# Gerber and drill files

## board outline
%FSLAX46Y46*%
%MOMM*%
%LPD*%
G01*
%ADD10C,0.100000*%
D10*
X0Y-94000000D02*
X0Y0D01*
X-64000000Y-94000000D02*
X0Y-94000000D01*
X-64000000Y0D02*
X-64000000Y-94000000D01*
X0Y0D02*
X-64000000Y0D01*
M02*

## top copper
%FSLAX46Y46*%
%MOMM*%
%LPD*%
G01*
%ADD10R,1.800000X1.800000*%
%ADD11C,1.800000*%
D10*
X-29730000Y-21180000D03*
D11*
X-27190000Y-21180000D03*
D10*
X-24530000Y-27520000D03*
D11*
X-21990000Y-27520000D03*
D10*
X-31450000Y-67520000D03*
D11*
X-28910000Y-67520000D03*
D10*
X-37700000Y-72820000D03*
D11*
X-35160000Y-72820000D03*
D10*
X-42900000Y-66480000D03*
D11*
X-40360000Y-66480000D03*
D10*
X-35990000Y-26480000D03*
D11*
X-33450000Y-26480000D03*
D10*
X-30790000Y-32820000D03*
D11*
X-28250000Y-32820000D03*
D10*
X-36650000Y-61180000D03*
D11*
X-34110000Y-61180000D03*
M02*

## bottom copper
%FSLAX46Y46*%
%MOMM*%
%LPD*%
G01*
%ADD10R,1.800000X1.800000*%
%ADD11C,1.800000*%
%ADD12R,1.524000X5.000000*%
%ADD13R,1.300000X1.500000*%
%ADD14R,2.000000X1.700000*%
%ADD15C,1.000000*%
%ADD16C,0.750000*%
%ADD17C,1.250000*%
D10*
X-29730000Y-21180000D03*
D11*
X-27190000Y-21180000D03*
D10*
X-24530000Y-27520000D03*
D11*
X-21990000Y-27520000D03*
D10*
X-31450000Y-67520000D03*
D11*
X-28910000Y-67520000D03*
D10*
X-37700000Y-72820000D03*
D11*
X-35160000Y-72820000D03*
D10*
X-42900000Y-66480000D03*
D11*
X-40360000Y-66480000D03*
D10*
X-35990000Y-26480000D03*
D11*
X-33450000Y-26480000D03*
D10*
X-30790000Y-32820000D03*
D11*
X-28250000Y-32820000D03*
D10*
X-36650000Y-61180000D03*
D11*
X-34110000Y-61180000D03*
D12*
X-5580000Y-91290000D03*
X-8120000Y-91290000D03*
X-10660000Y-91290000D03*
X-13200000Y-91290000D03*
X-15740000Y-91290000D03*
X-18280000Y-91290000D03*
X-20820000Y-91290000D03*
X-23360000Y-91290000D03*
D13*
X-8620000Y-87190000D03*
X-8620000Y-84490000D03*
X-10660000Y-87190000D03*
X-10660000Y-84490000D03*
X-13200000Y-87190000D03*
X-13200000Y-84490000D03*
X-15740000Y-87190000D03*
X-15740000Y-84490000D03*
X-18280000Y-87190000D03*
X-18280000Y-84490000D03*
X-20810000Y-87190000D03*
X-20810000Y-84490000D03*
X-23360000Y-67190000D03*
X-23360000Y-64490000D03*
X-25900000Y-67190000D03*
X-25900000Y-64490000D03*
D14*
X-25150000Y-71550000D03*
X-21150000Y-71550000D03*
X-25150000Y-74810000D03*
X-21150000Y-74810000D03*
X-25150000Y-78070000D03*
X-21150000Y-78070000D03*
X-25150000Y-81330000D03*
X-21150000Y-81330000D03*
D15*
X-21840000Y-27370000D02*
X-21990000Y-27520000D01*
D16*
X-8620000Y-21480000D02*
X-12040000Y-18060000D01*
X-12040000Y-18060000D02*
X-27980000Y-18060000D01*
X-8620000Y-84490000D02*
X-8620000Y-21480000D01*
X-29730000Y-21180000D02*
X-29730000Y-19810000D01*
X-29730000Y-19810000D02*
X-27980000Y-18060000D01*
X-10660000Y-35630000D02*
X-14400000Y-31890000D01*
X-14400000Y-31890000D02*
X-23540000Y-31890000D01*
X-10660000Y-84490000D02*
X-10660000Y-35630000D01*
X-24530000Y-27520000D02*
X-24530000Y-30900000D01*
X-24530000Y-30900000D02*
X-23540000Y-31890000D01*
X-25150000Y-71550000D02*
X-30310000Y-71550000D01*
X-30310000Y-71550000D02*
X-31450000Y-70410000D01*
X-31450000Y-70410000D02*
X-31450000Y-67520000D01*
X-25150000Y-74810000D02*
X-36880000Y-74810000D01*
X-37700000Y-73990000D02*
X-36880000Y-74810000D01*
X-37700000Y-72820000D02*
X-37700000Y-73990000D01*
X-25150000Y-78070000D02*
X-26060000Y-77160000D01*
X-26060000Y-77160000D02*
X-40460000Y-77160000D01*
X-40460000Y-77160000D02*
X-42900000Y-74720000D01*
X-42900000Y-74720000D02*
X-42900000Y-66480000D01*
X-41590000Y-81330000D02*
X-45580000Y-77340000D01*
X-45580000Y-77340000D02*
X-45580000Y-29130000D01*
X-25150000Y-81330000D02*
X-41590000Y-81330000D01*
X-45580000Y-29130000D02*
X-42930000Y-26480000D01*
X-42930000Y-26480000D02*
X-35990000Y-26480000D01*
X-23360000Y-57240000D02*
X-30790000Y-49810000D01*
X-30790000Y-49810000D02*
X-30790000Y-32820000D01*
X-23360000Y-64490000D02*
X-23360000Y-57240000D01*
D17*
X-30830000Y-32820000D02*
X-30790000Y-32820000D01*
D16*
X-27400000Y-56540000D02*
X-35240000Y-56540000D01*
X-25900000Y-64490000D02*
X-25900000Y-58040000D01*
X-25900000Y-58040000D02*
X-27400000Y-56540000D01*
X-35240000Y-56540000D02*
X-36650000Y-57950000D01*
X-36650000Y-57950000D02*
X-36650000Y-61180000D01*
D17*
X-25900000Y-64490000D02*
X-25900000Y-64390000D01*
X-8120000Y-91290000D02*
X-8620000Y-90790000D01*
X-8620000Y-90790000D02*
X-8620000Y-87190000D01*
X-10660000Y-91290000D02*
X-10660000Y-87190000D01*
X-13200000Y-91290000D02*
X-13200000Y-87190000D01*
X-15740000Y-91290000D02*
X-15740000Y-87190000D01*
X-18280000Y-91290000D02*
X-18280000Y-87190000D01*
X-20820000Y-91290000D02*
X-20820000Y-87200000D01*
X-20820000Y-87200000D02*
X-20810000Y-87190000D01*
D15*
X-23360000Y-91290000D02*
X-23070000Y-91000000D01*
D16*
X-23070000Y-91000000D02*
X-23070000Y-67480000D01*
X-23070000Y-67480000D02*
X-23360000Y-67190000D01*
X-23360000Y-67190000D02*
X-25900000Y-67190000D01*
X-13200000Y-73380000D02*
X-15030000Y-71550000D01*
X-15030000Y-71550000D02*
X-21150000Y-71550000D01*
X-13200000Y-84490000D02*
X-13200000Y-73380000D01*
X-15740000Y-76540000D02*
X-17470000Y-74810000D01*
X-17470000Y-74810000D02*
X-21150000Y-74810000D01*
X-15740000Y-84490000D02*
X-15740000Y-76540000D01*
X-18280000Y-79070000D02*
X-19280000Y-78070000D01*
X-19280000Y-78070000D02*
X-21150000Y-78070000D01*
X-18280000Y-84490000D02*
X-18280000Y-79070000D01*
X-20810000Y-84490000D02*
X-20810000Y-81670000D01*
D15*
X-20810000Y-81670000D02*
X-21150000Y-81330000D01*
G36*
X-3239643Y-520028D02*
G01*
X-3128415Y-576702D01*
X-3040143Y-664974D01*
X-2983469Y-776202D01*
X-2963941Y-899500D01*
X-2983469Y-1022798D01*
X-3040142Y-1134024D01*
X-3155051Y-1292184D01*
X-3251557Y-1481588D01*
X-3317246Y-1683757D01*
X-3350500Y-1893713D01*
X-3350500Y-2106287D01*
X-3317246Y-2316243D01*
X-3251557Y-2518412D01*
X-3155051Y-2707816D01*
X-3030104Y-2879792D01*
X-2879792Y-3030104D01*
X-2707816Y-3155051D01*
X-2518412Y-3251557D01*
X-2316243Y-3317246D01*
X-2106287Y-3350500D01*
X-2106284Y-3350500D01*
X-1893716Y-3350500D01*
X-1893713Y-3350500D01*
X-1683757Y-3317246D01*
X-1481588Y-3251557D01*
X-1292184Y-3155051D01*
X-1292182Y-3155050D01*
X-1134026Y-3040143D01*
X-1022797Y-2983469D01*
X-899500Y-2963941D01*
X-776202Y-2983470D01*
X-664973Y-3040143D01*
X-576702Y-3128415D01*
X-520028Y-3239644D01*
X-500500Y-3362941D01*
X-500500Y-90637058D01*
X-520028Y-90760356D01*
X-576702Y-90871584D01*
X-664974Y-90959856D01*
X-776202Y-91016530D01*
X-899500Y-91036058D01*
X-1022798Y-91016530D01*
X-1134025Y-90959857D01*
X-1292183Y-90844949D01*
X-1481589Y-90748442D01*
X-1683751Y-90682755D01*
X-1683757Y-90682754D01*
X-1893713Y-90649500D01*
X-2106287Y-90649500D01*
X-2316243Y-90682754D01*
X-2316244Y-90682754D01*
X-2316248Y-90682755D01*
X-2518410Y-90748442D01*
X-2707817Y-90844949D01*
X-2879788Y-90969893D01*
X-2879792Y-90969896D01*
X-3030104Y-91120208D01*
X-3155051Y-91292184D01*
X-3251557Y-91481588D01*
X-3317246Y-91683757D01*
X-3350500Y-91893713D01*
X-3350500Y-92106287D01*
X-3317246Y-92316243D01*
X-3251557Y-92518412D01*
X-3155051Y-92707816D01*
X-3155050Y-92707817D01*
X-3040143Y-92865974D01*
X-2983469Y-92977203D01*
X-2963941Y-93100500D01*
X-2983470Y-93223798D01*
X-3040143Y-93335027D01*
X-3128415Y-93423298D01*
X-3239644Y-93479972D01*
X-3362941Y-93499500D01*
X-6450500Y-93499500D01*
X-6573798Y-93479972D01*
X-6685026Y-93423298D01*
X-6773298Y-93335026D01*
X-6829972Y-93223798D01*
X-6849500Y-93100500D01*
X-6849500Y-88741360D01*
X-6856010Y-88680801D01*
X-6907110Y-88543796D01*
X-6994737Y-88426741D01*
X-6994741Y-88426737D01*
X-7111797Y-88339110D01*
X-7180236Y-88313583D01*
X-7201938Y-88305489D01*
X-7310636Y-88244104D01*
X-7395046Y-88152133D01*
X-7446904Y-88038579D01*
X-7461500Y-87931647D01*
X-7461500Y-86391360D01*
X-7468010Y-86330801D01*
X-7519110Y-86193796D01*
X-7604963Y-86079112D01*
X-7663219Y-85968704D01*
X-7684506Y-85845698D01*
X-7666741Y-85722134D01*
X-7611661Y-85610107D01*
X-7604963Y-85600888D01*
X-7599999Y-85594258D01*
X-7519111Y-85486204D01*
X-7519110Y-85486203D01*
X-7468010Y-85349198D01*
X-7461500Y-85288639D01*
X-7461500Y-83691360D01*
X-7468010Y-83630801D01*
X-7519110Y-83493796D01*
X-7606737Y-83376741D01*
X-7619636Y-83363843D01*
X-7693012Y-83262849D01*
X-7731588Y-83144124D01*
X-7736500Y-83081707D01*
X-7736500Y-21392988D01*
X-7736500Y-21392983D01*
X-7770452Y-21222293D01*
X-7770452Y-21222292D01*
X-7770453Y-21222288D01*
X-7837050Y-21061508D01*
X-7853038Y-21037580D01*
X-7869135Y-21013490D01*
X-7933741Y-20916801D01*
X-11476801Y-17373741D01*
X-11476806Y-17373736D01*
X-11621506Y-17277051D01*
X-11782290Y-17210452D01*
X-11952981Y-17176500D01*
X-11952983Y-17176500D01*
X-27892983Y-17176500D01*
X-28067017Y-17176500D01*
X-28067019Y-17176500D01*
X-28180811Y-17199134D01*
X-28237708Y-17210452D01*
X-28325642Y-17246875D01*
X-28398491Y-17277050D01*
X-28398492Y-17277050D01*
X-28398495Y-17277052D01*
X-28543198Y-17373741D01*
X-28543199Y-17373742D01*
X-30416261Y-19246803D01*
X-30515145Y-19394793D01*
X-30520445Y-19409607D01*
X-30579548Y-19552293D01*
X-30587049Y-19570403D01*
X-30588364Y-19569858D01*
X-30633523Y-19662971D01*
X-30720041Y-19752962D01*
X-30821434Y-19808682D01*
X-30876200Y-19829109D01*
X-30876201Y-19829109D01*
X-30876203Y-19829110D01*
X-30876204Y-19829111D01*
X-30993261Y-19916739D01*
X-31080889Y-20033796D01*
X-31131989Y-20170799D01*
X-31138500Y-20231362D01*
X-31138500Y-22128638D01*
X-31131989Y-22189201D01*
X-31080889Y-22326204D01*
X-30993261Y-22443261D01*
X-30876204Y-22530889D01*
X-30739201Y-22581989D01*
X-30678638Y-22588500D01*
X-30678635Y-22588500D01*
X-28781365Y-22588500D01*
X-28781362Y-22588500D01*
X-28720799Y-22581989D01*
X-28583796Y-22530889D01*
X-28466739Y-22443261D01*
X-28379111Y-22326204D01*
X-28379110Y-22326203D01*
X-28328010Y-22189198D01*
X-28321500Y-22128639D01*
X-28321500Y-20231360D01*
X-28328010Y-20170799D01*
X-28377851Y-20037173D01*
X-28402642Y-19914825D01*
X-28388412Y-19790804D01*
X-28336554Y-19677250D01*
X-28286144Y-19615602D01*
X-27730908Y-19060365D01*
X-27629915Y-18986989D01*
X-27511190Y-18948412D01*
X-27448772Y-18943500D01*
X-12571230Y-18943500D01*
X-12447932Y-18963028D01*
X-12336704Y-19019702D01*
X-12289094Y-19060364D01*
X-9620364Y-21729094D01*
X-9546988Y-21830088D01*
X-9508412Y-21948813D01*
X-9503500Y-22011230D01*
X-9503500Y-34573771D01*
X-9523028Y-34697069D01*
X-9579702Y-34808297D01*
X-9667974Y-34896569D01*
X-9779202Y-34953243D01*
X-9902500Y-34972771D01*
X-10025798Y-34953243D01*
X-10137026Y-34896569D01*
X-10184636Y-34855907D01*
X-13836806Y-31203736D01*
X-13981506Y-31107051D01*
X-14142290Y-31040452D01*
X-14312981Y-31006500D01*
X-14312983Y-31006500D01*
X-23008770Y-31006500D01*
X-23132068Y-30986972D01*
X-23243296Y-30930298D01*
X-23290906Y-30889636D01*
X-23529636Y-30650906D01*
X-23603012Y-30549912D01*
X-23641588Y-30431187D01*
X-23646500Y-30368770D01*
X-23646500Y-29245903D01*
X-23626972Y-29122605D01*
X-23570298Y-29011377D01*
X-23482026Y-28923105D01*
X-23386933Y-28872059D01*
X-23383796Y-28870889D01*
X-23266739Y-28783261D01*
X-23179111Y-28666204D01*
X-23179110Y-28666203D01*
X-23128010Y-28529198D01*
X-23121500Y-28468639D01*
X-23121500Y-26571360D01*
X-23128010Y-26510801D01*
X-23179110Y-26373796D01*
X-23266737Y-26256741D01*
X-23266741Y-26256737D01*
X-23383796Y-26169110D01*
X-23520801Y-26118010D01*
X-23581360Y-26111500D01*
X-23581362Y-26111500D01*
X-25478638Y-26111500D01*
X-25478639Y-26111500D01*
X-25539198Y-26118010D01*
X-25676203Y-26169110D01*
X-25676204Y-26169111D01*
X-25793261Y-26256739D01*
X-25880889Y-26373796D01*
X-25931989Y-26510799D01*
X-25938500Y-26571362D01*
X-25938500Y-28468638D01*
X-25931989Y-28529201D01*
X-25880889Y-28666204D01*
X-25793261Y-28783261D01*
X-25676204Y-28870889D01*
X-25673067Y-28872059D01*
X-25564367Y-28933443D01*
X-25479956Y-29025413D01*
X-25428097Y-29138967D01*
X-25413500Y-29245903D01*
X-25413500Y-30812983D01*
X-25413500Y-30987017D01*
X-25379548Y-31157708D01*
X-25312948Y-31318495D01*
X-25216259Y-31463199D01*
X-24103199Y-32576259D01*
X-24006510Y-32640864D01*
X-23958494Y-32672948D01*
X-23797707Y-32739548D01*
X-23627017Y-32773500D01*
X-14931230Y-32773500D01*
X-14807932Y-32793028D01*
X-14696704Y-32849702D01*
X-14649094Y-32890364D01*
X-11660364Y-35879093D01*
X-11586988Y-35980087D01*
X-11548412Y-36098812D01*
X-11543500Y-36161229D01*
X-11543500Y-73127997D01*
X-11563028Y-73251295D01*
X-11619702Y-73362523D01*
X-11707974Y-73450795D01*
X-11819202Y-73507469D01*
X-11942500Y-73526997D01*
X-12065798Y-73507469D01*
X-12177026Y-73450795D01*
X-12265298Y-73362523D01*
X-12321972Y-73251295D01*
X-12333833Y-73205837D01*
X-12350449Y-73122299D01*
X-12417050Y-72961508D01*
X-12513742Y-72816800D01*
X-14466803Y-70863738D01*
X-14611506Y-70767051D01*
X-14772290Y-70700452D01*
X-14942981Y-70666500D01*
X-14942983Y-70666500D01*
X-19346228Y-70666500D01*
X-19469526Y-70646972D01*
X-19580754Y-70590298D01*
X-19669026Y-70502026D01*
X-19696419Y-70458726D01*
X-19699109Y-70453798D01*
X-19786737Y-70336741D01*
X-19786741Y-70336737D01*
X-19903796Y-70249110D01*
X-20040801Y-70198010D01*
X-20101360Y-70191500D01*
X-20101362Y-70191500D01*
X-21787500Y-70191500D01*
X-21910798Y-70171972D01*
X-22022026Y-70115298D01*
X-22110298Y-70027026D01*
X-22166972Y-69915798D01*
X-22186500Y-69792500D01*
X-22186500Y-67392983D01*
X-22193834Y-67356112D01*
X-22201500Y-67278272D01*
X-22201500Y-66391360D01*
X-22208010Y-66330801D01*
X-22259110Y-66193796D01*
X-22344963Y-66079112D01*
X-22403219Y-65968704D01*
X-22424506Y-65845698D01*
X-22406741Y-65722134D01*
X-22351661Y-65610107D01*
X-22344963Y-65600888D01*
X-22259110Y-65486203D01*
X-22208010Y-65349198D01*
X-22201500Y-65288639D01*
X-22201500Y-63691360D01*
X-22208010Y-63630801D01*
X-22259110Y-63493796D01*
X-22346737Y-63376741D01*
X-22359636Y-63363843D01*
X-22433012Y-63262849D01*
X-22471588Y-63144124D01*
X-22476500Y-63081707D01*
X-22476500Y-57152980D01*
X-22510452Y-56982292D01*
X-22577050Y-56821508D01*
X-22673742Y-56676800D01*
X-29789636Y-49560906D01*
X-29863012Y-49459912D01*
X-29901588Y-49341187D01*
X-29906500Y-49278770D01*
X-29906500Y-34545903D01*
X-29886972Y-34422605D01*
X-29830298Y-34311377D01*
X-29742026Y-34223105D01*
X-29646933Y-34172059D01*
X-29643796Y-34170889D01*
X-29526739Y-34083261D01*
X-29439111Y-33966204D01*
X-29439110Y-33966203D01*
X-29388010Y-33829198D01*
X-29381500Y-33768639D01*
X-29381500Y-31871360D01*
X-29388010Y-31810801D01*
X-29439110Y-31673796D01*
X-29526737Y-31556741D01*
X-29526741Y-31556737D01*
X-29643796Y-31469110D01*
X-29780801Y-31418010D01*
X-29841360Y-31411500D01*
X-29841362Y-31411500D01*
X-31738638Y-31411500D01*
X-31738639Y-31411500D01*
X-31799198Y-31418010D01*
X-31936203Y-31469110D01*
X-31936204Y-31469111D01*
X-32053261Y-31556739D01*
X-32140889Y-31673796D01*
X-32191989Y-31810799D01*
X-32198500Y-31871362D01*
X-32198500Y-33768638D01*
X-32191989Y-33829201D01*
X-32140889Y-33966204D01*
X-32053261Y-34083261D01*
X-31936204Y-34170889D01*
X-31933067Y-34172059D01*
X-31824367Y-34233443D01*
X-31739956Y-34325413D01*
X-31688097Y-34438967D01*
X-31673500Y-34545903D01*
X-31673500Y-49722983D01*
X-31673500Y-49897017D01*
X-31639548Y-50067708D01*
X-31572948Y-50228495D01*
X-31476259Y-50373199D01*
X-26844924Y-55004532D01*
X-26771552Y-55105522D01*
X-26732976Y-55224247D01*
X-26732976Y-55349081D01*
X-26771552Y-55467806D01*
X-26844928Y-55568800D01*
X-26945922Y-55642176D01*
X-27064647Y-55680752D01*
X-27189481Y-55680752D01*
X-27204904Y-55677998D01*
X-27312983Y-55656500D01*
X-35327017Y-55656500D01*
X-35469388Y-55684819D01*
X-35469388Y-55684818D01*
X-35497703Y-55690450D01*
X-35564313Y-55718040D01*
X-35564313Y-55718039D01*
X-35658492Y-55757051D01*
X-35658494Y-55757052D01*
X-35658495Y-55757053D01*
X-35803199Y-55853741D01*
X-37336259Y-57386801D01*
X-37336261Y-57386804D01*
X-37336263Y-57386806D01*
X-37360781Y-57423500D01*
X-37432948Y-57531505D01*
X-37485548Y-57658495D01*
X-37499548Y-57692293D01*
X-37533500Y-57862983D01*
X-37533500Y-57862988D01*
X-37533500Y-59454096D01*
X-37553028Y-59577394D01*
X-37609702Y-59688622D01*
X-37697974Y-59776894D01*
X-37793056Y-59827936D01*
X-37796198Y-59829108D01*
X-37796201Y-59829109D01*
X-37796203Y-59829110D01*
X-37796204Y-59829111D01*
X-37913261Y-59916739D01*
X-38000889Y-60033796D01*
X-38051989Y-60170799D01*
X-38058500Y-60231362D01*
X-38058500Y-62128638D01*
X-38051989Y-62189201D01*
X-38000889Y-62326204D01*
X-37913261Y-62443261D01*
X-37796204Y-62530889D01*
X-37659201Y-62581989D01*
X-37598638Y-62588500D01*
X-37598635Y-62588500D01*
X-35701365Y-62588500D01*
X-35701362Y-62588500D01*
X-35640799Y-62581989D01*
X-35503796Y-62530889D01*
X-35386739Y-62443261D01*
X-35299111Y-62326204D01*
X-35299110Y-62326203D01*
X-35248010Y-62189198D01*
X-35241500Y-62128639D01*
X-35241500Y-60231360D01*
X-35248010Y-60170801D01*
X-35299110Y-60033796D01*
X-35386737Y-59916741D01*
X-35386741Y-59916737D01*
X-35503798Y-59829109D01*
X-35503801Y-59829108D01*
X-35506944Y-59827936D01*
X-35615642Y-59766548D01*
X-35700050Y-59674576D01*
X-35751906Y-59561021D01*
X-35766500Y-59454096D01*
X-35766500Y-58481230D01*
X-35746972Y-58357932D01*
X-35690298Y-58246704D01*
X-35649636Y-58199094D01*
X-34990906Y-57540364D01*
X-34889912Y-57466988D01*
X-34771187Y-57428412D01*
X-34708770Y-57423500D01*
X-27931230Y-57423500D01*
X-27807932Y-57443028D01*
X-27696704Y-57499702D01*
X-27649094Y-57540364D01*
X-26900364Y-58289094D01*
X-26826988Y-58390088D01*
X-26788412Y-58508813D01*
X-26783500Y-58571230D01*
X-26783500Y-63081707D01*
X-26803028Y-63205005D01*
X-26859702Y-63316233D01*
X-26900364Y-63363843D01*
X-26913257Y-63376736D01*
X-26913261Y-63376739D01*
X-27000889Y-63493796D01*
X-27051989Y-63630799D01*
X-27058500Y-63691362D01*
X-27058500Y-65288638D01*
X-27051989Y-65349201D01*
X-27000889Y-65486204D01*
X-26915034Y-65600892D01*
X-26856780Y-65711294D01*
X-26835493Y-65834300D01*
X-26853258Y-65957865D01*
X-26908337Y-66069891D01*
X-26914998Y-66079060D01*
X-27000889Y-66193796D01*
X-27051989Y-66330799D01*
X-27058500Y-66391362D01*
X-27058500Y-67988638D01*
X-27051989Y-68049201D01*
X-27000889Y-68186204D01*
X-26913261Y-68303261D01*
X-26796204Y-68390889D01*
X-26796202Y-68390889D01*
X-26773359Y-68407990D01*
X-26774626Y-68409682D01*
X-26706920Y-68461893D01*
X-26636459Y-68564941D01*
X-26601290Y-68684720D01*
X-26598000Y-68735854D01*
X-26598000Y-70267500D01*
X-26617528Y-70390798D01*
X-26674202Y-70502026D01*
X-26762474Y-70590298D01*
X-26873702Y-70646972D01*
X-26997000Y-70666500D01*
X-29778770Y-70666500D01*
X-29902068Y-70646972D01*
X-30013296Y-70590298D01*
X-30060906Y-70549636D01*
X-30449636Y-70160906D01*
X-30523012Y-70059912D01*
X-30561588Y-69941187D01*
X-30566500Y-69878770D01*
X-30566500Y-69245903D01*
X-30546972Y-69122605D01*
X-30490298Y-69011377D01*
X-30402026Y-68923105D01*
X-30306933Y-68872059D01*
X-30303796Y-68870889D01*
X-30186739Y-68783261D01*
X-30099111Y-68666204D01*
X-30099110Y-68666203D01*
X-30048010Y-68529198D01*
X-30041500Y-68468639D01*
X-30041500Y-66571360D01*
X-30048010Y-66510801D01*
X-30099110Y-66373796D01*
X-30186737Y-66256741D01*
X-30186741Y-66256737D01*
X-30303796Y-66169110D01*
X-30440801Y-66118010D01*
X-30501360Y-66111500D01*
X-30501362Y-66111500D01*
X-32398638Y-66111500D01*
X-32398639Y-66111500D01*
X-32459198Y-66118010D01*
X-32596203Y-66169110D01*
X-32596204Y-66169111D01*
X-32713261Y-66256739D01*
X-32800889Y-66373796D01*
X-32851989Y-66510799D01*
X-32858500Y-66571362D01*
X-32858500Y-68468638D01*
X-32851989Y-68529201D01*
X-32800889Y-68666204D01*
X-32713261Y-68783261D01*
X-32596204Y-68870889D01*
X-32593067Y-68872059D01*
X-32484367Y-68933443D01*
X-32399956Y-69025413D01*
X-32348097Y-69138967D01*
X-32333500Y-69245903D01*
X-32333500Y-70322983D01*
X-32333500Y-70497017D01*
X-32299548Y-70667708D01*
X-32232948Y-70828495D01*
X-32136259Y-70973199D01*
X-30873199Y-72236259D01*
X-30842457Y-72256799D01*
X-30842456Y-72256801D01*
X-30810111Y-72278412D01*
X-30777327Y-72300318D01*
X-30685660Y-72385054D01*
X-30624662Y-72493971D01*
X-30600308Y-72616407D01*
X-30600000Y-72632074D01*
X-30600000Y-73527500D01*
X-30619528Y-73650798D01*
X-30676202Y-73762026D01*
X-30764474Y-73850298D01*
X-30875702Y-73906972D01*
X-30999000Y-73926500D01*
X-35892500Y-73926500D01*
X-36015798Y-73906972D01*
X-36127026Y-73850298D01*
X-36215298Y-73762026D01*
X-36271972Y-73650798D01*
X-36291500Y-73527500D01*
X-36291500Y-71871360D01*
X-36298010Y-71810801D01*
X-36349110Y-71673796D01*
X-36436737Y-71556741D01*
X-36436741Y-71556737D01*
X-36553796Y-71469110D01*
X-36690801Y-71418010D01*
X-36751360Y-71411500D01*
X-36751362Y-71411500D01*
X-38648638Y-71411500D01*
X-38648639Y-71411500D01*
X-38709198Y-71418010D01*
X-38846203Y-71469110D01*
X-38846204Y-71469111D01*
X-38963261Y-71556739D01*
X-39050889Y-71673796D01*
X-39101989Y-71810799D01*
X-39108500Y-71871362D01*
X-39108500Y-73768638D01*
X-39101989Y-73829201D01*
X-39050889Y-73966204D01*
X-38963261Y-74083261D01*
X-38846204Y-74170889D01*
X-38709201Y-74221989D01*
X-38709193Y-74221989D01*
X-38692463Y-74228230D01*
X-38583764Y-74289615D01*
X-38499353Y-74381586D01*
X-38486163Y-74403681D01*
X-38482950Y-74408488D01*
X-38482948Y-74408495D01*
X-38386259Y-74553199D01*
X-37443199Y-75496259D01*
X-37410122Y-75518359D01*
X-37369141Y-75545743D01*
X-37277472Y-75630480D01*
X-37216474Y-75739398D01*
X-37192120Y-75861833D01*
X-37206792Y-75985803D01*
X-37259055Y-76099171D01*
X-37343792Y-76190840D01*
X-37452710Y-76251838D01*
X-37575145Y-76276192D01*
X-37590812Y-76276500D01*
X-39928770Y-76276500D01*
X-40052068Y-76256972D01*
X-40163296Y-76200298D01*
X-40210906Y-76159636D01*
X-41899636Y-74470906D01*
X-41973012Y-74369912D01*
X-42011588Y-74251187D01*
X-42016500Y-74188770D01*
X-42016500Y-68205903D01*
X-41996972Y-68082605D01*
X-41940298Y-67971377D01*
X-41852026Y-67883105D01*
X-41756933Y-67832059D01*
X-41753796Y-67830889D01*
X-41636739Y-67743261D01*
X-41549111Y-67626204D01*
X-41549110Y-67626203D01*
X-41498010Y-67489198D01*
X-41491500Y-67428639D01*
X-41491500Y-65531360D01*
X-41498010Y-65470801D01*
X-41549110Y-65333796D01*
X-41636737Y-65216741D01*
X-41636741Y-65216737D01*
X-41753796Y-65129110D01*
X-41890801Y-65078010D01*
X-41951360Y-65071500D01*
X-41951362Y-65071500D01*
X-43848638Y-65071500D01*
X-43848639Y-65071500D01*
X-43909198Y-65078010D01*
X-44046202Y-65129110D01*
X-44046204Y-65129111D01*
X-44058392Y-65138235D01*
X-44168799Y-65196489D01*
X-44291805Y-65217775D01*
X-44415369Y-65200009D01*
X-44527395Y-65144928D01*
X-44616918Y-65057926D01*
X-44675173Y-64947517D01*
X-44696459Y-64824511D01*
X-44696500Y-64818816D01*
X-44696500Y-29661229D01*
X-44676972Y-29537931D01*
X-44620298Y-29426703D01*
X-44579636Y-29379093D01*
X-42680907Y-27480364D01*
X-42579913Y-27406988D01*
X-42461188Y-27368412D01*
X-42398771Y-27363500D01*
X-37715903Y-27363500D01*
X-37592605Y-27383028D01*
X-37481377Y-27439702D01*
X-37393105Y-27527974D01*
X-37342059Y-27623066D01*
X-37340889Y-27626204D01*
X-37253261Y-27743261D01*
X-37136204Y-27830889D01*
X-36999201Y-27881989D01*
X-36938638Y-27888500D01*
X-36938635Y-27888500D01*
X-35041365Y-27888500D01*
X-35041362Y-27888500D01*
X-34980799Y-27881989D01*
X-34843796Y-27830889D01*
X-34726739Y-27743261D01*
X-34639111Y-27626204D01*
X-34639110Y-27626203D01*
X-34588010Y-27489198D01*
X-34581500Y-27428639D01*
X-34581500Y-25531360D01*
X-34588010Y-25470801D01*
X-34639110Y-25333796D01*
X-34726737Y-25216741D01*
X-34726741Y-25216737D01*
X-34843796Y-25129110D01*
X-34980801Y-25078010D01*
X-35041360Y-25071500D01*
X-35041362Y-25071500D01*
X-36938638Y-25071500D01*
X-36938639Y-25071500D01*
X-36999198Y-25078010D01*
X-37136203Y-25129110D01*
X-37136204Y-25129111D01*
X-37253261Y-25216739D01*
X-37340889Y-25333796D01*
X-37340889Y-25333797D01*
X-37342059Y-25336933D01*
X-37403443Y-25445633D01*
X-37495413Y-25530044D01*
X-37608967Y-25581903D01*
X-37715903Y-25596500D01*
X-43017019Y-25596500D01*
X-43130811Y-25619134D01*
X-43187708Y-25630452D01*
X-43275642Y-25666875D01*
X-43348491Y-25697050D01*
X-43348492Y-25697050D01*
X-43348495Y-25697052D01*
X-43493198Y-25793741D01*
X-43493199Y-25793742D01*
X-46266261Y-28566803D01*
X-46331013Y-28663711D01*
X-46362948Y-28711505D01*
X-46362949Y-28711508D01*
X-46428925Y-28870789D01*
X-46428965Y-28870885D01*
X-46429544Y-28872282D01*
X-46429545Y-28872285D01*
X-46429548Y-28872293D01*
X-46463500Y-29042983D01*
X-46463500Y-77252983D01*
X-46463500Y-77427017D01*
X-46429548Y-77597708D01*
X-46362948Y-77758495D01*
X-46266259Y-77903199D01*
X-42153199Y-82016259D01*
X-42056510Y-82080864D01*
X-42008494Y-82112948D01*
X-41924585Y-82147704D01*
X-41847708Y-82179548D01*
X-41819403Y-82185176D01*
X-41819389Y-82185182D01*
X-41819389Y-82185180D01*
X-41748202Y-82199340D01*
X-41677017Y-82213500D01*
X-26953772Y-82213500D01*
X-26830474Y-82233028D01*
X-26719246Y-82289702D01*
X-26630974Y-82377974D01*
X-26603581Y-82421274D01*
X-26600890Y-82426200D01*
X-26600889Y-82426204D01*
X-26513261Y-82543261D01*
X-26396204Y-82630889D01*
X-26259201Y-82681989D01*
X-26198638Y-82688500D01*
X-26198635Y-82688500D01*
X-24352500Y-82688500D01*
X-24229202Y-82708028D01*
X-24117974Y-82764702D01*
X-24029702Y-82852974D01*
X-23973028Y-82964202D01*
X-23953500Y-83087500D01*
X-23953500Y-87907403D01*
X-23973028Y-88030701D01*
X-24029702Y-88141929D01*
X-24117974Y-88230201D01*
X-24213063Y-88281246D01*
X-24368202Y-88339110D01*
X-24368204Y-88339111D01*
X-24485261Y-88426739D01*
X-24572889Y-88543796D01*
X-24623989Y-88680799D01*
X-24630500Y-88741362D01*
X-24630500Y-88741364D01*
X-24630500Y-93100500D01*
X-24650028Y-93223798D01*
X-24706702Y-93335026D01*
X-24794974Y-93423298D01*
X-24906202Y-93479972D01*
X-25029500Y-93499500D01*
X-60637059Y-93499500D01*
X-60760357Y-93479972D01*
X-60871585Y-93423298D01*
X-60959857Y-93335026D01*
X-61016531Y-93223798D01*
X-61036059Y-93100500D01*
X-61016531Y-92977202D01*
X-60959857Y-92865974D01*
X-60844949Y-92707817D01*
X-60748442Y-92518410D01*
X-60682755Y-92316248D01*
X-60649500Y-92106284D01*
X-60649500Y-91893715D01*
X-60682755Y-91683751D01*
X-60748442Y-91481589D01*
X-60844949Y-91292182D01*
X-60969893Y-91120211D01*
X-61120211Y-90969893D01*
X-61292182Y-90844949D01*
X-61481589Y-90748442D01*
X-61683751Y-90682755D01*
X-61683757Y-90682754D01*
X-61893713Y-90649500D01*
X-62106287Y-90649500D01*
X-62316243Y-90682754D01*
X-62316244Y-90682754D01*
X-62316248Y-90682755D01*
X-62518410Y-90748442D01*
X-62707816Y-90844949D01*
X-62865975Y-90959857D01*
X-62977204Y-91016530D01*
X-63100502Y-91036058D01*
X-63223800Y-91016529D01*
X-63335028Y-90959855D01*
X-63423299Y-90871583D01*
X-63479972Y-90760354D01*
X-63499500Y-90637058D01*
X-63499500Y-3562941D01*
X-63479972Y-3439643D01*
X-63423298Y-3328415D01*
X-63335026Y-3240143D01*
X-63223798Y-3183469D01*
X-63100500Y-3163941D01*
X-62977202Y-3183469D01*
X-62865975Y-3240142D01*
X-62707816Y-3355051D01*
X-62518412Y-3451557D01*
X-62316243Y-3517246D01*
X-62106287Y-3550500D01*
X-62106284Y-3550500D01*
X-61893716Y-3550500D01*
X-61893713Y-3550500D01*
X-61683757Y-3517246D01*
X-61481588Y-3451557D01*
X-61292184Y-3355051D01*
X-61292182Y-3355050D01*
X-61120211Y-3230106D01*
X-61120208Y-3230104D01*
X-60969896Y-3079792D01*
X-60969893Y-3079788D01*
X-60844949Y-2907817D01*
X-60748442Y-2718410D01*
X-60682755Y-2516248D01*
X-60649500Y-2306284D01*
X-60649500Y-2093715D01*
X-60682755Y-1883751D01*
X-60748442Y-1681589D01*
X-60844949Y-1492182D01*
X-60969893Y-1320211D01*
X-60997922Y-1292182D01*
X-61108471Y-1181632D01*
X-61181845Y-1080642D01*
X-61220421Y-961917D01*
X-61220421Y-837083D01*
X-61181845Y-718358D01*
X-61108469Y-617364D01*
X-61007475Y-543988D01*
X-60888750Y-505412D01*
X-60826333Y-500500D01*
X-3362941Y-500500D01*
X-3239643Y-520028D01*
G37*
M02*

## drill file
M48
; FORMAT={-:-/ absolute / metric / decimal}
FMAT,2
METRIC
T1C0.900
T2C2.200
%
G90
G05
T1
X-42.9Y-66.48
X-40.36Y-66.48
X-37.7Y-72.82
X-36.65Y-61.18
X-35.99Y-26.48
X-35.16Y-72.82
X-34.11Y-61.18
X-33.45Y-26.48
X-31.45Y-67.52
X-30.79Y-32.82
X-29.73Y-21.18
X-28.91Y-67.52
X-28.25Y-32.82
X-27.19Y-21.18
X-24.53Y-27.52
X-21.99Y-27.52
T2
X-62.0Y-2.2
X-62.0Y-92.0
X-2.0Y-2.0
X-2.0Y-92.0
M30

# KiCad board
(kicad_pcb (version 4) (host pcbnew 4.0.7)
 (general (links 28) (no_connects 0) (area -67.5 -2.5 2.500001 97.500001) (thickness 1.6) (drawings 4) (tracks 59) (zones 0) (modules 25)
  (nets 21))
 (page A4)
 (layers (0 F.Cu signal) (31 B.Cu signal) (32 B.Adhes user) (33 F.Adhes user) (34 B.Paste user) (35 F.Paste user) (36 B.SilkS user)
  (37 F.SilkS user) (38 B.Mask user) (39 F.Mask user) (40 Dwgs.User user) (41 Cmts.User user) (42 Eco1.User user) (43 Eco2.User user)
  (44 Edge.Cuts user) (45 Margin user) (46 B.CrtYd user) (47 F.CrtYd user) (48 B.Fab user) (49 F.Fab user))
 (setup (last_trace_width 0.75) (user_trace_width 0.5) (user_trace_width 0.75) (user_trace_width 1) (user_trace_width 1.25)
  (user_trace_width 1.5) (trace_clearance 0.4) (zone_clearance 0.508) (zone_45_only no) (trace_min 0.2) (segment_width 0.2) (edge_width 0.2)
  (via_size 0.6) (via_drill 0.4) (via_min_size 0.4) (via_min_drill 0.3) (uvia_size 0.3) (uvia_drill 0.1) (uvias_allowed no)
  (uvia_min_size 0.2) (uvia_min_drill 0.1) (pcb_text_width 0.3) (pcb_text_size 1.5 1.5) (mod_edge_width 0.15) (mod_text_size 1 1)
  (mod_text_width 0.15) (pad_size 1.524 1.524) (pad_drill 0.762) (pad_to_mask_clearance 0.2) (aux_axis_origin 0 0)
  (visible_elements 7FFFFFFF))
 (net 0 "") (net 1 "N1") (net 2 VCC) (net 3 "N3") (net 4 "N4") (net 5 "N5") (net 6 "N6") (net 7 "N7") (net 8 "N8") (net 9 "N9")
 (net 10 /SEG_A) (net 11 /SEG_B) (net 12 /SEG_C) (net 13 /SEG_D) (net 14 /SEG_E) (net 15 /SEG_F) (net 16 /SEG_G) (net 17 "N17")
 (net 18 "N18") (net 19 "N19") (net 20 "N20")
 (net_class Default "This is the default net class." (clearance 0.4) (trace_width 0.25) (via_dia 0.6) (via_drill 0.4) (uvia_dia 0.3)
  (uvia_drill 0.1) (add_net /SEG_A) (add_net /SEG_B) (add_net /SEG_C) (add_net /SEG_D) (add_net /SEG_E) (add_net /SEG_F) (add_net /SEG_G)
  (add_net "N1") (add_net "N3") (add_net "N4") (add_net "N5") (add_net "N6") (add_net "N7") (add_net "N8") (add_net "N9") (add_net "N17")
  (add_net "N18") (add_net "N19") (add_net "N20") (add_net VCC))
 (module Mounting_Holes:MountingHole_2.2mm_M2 (layer F.Cu) (at -2 92)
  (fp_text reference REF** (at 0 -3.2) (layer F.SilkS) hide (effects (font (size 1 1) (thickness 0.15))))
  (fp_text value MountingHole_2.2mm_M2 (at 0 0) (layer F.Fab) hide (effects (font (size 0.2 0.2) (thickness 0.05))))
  (pad 1 np_thru_hole circle (at 0 0) (size 2.2 2.2) (drill 2.2) (layers *.Cu *.Mask)))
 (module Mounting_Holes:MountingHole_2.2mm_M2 (layer F.Cu) (at -62 92)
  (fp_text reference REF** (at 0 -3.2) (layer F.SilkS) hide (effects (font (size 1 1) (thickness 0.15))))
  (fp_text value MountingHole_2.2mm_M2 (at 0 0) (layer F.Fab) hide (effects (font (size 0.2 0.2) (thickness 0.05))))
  (pad 1 np_thru_hole circle (at 0 0) (size 2.2 2.2) (drill 2.2) (layers *.Cu *.Mask)))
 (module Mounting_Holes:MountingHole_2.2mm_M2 (layer F.Cu) (at -2 2)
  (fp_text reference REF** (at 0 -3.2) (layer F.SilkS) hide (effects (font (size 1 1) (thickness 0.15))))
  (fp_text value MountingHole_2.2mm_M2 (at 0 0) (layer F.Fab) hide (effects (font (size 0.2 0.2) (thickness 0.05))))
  (pad 1 np_thru_hole circle (at 0 0) (size 2.2 2.2) (drill 2.2) (layers *.Cu *.Mask)))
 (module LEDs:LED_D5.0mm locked (layer F.Cu) (at -29.73 21.18)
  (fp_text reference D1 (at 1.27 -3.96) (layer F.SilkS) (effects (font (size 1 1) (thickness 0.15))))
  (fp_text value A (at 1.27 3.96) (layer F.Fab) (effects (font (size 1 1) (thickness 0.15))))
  (pad 1 thru_hole rect (at 0 0) (size 1.8 1.8) (drill 0.9) (layers *.Cu *.Mask) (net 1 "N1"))
  (pad 2 thru_hole circle (at 2.54 0) (size 1.8 1.8) (drill 0.9) (layers *.Cu *.Mask) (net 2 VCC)))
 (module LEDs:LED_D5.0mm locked (layer F.Cu) (at -24.53 27.52)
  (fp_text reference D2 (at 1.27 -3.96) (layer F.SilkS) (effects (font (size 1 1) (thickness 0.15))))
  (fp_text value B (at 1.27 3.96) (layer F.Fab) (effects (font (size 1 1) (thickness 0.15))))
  (pad 1 thru_hole rect (at 0 0) (size 1.8 1.8) (drill 0.9) (layers *.Cu *.Mask) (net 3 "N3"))
  (pad 2 thru_hole circle (at 2.54 0) (size 1.8 1.8) (drill 0.9) (layers *.Cu *.Mask) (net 2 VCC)))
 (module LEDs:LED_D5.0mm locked (layer F.Cu) (at -31.45 67.52)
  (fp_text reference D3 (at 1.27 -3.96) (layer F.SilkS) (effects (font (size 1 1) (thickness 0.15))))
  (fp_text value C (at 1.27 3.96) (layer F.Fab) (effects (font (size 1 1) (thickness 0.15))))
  (pad 1 thru_hole rect (at 0 0) (size 1.8 1.8) (drill 0.9) (layers *.Cu *.Mask) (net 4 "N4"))
  (pad 2 thru_hole circle (at 2.54 0) (size 1.8 1.8) (drill 0.9) (layers *.Cu *.Mask) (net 2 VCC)))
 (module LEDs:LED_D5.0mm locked (layer F.Cu) (at -37.7 72.82)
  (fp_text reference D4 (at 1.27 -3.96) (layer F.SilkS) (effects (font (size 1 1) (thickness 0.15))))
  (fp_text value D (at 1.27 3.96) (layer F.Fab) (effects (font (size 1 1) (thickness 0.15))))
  (pad 1 thru_hole rect (at 0 0) (size 1.8 1.8) (drill 0.9) (layers *.Cu *.Mask) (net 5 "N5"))
  (pad 2 thru_hole circle (at 2.54 0) (size 1.8 1.8) (drill 0.9) (layers *.Cu *.Mask) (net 2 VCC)))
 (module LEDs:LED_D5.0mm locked (layer F.Cu) (at -42.9 66.48)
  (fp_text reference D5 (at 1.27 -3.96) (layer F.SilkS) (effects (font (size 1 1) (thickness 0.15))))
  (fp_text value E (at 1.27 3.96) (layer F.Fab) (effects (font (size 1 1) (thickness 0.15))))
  (pad 1 thru_hole rect (at 0 0) (size 1.8 1.8) (drill 0.9) (layers *.Cu *.Mask) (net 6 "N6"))
  (pad 2 thru_hole circle (at 2.54 0) (size 1.8 1.8) (drill 0.9) (layers *.Cu *.Mask) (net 2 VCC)))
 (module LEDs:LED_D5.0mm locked (layer F.Cu) (at -35.99 26.48)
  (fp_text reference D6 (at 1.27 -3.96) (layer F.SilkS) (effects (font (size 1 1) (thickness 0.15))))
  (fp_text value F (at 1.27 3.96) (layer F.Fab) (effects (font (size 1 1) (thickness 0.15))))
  (pad 1 thru_hole rect (at 0 0) (size 1.8 1.8) (drill 0.9) (layers *.Cu *.Mask) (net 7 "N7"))
  (pad 2 thru_hole circle (at 2.54 0) (size 1.8 1.8) (drill 0.9) (layers *.Cu *.Mask) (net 2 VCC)))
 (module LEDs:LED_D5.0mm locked (layer F.Cu) (at -30.79 32.82)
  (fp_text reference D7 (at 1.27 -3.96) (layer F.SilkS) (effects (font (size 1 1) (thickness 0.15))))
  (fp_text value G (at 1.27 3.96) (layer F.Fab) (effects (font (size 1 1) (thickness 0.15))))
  (pad 1 thru_hole rect (at 0 0) (size 1.8 1.8) (drill 0.9) (layers *.Cu *.Mask) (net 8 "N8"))
  (pad 2 thru_hole circle (at 2.54 0) (size 1.8 1.8) (drill 0.9) (layers *.Cu *.Mask) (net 2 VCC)))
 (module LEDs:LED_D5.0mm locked (layer F.Cu) (at -36.65 61.18)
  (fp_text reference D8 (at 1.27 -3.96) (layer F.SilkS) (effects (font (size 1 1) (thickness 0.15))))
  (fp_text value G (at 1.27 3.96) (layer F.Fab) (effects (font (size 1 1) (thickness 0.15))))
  (pad 1 thru_hole rect (at 0 0) (size 1.8 1.8) (drill 0.9) (layers *.Cu *.Mask) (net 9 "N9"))
  (pad 2 thru_hole circle (at 2.54 0) (size 1.8 1.8) (drill 0.9) (layers *.Cu *.Mask) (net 2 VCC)))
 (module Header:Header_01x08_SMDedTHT (layer B.Cu) (at -5.58 91.29 90)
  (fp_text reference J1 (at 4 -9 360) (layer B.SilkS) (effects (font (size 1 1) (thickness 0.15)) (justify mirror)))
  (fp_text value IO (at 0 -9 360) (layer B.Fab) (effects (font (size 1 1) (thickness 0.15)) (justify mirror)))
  (pad 1 smd rect (at 0 0 90) (size 5 1.524) (layers B.Cu B.Paste B.Mask) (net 2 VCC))
  (pad 2 smd rect (at 0 -2.54 90) (size 5 1.524) (layers B.Cu B.Paste B.Mask) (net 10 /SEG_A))
  (pad 3 smd rect (at 0 -5.08 90) (size 5 1.524) (layers B.Cu B.Paste B.Mask) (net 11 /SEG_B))
  (pad 4 smd rect (at 0 -7.62 90) (size 5 1.524) (layers B.Cu B.Paste B.Mask) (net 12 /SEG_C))
  (pad 5 smd rect (at 0 -10.16 90) (size 5 1.524) (layers B.Cu B.Paste B.Mask) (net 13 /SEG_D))
  (pad 6 smd rect (at 0 -12.7 90) (size 5 1.524) (layers B.Cu B.Paste B.Mask) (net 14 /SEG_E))
  (pad 7 smd rect (at 0 -15.24 90) (size 5 1.524) (layers B.Cu B.Paste B.Mask) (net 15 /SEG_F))
  (pad 8 smd rect (at 0 -17.78 90) (size 5 1.524) (layers B.Cu B.Paste B.Mask) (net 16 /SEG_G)))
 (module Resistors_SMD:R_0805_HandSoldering (layer B.Cu) (at -8.62 85.84 90)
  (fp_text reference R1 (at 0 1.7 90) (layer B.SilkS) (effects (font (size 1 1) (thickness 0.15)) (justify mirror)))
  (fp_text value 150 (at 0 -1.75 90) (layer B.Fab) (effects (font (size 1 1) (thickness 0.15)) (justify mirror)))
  (pad 1 smd rect (at -1.35 0 90) (size 1.5 1.3) (layers B.Cu B.Paste B.Mask) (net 10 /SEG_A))
  (pad 2 smd rect (at 1.35 0 90) (size 1.5 1.3) (layers B.Cu B.Paste B.Mask) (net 1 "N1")))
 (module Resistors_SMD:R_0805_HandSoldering (layer B.Cu) (at -10.66 85.84 90)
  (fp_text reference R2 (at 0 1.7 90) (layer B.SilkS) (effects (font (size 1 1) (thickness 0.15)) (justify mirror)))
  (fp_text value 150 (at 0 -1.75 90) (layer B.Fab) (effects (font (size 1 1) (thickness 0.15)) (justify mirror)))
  (pad 1 smd rect (at -1.35 0 90) (size 1.5 1.3) (layers B.Cu B.Paste B.Mask) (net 11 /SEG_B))
  (pad 2 smd rect (at 1.35 0 90) (size 1.5 1.3) (layers B.Cu B.Paste B.Mask) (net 3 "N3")))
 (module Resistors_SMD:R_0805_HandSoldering (layer B.Cu) (at -13.2 85.84 90)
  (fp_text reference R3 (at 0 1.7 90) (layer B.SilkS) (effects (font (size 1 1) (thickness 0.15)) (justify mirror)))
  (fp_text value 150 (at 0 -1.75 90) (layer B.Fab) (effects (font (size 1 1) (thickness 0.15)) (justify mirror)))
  (pad 1 smd rect (at -1.35 0 90) (size 1.5 1.3) (layers B.Cu B.Paste B.Mask) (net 12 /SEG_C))
  (pad 2 smd rect (at 1.35 0 90) (size 1.5 1.3) (layers B.Cu B.Paste B.Mask) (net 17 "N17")))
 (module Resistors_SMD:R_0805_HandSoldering (layer B.Cu) (at -15.74 85.84 90)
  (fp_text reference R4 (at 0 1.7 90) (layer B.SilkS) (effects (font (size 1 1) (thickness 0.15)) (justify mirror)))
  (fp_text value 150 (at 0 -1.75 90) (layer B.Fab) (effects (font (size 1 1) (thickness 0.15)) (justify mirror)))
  (pad 1 smd rect (at -1.35 0 90) (size 1.5 1.3) (layers B.Cu B.Paste B.Mask) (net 13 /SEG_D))
  (pad 2 smd rect (at 1.35 0 90) (size 1.5 1.3) (layers B.Cu B.Paste B.Mask) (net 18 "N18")))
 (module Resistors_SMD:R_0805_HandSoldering (layer B.Cu) (at -18.28 85.84 90)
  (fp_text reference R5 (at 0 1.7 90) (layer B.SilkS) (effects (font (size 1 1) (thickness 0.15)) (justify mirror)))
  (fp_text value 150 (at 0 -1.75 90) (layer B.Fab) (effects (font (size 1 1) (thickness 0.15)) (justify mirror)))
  (pad 1 smd rect (at -1.35 0 90) (size 1.5 1.3) (layers B.Cu B.Paste B.Mask) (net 14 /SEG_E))
  (pad 2 smd rect (at 1.35 0 90) (size 1.5 1.3) (layers B.Cu B.Paste B.Mask) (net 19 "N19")))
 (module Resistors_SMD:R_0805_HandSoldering (layer B.Cu) (at -20.81 85.84 90)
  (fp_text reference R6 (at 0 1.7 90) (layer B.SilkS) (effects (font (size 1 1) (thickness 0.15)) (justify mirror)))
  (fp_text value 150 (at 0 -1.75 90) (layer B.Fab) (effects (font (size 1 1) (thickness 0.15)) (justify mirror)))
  (pad 1 smd rect (at -1.35 0 90) (size 1.5 1.3) (layers B.Cu B.Paste B.Mask) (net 15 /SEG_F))
  (pad 2 smd rect (at 1.35 0 90) (size 1.5 1.3) (layers B.Cu B.Paste B.Mask) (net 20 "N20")))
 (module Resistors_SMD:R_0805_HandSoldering (layer B.Cu) (at -23.36 65.84 90)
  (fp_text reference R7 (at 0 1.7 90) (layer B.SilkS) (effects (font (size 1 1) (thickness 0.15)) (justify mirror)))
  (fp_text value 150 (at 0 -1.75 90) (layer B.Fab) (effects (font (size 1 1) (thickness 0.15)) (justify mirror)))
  (pad 1 smd rect (at -1.35 0 90) (size 1.5 1.3) (layers B.Cu B.Paste B.Mask) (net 16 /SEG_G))
  (pad 2 smd rect (at 1.35 0 90) (size 1.5 1.3) (layers B.Cu B.Paste B.Mask) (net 8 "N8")))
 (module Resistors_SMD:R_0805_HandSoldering (layer B.Cu) (at -25.9 65.84 90)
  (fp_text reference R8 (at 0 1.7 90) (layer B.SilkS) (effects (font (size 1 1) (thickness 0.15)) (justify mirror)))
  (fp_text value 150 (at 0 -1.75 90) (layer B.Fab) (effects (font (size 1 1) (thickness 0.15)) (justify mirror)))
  (pad 1 smd rect (at -1.35 0 90) (size 1.5 1.3) (layers B.Cu B.Paste B.Mask) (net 16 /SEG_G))
  (pad 2 smd rect (at 1.35 0 90) (size 1.5 1.3) (layers B.Cu B.Paste B.Mask) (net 9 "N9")))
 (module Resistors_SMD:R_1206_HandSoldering (layer B.Cu) (at -23.15 71.55)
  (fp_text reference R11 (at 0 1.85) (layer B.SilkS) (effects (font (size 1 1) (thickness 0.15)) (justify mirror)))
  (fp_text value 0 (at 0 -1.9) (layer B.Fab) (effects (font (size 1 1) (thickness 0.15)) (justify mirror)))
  (pad 1 smd rect (at -2 0) (size 2 1.7) (layers B.Cu B.Paste B.Mask) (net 4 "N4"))
  (pad 2 smd rect (at 2 0) (size 2 1.7) (layers B.Cu B.Paste B.Mask) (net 17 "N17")))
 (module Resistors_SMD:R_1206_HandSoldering (layer B.Cu) (at -23.15 74.81)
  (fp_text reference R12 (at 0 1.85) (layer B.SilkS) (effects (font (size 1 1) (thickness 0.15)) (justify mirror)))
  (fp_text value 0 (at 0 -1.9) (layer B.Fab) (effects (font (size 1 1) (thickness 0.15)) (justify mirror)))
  (pad 1 smd rect (at -2 0) (size 2 1.7) (layers B.Cu B.Paste B.Mask) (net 5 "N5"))
  (pad 2 smd rect (at 2 0) (size 2 1.7) (layers B.Cu B.Paste B.Mask) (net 18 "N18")))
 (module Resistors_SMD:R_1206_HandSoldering (layer B.Cu) (at -23.15 78.07)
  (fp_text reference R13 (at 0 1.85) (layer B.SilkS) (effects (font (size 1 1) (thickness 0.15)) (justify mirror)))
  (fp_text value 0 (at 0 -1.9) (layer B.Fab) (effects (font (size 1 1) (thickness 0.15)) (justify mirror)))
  (pad 1 smd rect (at -2 0) (size 2 1.7) (layers B.Cu B.Paste B.Mask) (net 6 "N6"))
  (pad 2 smd rect (at 2 0) (size 2 1.7) (layers B.Cu B.Paste B.Mask) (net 19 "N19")))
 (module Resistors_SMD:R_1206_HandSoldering (layer B.Cu) (at -23.15 81.33)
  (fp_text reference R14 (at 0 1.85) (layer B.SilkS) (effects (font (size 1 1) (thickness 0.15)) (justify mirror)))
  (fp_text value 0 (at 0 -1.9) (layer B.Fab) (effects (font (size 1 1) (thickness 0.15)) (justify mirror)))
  (pad 1 smd rect (at -2 0) (size 2 1.7) (layers B.Cu B.Paste B.Mask) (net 7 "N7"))
  (pad 2 smd rect (at 2 0) (size 2 1.7) (layers B.Cu B.Paste B.Mask) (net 20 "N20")))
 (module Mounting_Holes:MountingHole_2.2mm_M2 (layer F.Cu) (at -62 2.2)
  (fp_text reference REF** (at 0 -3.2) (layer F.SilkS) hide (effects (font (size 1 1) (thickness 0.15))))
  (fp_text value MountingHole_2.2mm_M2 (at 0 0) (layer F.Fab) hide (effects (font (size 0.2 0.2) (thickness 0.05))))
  (pad 1 np_thru_hole circle (at 0 0) (size 2.2 2.2) (drill 2.2) (layers *.Cu *.Mask)))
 (gr_line (start 0 94) (end 0 0) (layer Edge.Cuts) (width 0.1))
 (gr_line (start -64 94) (end 0 94) (layer Edge.Cuts) (width 0.1))
 (gr_line (start -64 0) (end -64 94) (layer Edge.Cuts) (width 0.1))
 (gr_line (start 0 0) (end -64 0) (layer Edge.Cuts) (width 0.1))
 (segment (start -21.84 27.37) (end -21.99 27.52) (width 1) (layer B.Cu) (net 2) (status 30))
 (segment (start -8.62 21.48) (end -12.04 18.06) (width 0.75) (layer B.Cu) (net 1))
 (segment (start -12.04 18.06) (end -27.98 18.06) (width 0.75) (layer B.Cu) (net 1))
 (segment (start -8.62 84.49) (end -8.62 21.48) (width 0.75) (layer B.Cu) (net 1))
 (segment (start -29.73 21.18) (end -29.73 19.81) (width 0.75) (layer B.Cu) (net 1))
 (segment (start -29.73 19.81) (end -27.98 18.06) (width 0.75) (layer B.Cu) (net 1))
 (segment (start -10.66 35.63) (end -14.4 31.89) (width 0.75) (layer B.Cu) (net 3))
 (segment (start -14.4 31.89) (end -23.54 31.89) (width 0.75) (layer B.Cu) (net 3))
 (segment (start -10.66 84.49) (end -10.66 35.63) (width 0.75) (layer B.Cu) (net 3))
 (segment (start -24.53 27.52) (end -24.53 30.9) (width 0.75) (layer B.Cu) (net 3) (status 10))
 (segment (start -24.53 30.9) (end -23.54 31.89) (width 0.75) (layer B.Cu) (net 3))
 (segment (start -25.15 71.55) (end -30.31 71.55) (width 0.75) (layer B.Cu) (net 4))
 (segment (start -30.31 71.55) (end -31.45 70.41) (width 0.75) (layer B.Cu) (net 4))
 (segment (start -31.45 70.41) (end -31.45 67.52) (width 0.75) (layer B.Cu) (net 4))
 (segment (start -25.15 74.81) (end -36.88 74.81) (width 0.75) (layer B.Cu) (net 5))
 (segment (start -37.7 73.99) (end -36.88 74.81) (width 0.75) (layer B.Cu) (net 5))
 (segment (start -37.7 72.82) (end -37.7 73.99) (width 0.75) (layer B.Cu) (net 5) (status 10))
 (segment (start -25.15 78.07) (end -26.06 77.16) (width 0.75) (layer B.Cu) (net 6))
 (segment (start -26.06 77.16) (end -40.46 77.16) (width 0.75) (layer B.Cu) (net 6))
 (segment (start -40.46 77.16) (end -42.9 74.72) (width 0.75) (layer B.Cu) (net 6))
 (segment (start -42.9 74.72) (end -42.9 66.48) (width 0.75) (layer B.Cu) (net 6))
 (segment (start -41.59 81.33) (end -45.58 77.34) (width 0.75) (layer B.Cu) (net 7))
 (segment (start -45.58 77.34) (end -45.58 29.13) (width 0.75) (layer B.Cu) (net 7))
 (segment (start -25.15 81.33) (end -41.59 81.33) (width 0.75) (layer B.Cu) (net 7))
 (segment (start -45.58 29.13) (end -42.93 26.48) (width 0.75) (layer B.Cu) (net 7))
 (segment (start -42.93 26.48) (end -35.99 26.48) (width 0.75) (layer B.Cu) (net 7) (status 20))
 (segment (start -23.36 57.24) (end -30.79 49.81) (width 0.75) (layer B.Cu) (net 8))
 (segment (start -30.79 49.81) (end -30.79 32.82) (width 0.75) (layer B.Cu) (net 8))
 (segment (start -23.36 64.49) (end -23.36 57.24) (width 0.75) (layer B.Cu) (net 8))
 (segment (start -30.83 32.82) (end -30.79 32.82) (width 1.25) (layer B.Cu) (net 8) (status 30))
 (segment (start -27.4 56.54) (end -35.24 56.54) (width 0.75) (layer B.Cu) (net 9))
 (segment (start -25.9 64.49) (end -25.9 58.04) (width 0.75) (layer B.Cu) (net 9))
 (segment (start -25.9 58.04) (end -27.4 56.54) (width 0.75) (layer B.Cu) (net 9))
 (segment (start -35.24 56.54) (end -36.65 57.95) (width 0.75) (layer B.Cu) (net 9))
 (segment (start -36.65 57.95) (end -36.65 61.18) (width 0.75) (layer B.Cu) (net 9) (status 20))
 (segment (start -25.9 64.49) (end -25.9 64.39) (width 1.25) (layer B.Cu) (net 9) (status 30))
 (segment (start -8.12 91.29) (end -8.62 90.79) (width 1.25) (layer B.Cu) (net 10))
 (segment (start -8.62 90.79) (end -8.62 87.19) (width 1.25) (layer B.Cu) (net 10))
 (segment (start -10.66 91.29) (end -10.66 87.19) (width 1.25) (layer B.Cu) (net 11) (status 30))
 (segment (start -13.2 91.29) (end -13.2 87.19) (width 1.25) (layer B.Cu) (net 12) (status 30))
 (segment (start -15.74 91.29) (end -15.74 87.19) (width 1.25) (layer B.Cu) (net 13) (status 30))
 (segment (start -18.28 91.29) (end -18.28 87.19) (width 1.25) (layer B.Cu) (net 14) (status 30))
 (segment (start -20.82 91.29) (end -20.82 87.2) (width 1.25) (layer B.Cu) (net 15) (status 30))
 (segment (start -20.82 87.2) (end -20.81 87.19) (width 1.25) (layer B.Cu) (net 15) (status 30))
 (segment (start -23.36 91.29) (end -23.07 91) (width 1) (layer B.Cu) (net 16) (status 30))
 (segment (start -23.07 91) (end -23.07 67.48) (width 0.75) (layer B.Cu) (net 16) (status 30))
 (segment (start -23.07 67.48) (end -23.36 67.19) (width 0.75) (layer B.Cu) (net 16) (status 30))
 (segment (start -23.36 67.19) (end -25.9 67.19) (width 0.75) (layer B.Cu) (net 16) (status 30))
 (segment (start -13.2 73.38) (end -15.03 71.55) (width 0.75) (layer B.Cu) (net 17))
 (segment (start -15.03 71.55) (end -21.15 71.55) (width 0.75) (layer B.Cu) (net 17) (status 20))
 (segment (start -13.2 84.49) (end -13.2 73.38) (width 0.75) (layer B.Cu) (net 17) (status 10))
 (segment (start -15.74 76.54) (end -17.47 74.81) (width 0.75) (layer B.Cu) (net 18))
 (segment (start -17.47 74.81) (end -21.15 74.81) (width 0.75) (layer B.Cu) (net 18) (status 20))
 (segment (start -15.74 84.49) (end -15.74 76.54) (width 0.75) (layer B.Cu) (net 18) (status 10))
 (segment (start -18.28 79.07) (end -19.28 78.07) (width 0.75) (layer B.Cu) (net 19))
 (segment (start -19.28 78.07) (end -21.15 78.07) (width 0.75) (layer B.Cu) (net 19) (status 20))
 (segment (start -18.28 84.49) (end -18.28 79.07) (width 0.75) (layer B.Cu) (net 19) (status 10))
 (segment (start -20.81 84.49) (end -20.81 81.67) (width 0.75) (layer B.Cu) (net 20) (status 30))
 (segment (start -20.81 81.67) (end -21.15 81.33) (width 1) (layer B.Cu) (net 20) (status 30))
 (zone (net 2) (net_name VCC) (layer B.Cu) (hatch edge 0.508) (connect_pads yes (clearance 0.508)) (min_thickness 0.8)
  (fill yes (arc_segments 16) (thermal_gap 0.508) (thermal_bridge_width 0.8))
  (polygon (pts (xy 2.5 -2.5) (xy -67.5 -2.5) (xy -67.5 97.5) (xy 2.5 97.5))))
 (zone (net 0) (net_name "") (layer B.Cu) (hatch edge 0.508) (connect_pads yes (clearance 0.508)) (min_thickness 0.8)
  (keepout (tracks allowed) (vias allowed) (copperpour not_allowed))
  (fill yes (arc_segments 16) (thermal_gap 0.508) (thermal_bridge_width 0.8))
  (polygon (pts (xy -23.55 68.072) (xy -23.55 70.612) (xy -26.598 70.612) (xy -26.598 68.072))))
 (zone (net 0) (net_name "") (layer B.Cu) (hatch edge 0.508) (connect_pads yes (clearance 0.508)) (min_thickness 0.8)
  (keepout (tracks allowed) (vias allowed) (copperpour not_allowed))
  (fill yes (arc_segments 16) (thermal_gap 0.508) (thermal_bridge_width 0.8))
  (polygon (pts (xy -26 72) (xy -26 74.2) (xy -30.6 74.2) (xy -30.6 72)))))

